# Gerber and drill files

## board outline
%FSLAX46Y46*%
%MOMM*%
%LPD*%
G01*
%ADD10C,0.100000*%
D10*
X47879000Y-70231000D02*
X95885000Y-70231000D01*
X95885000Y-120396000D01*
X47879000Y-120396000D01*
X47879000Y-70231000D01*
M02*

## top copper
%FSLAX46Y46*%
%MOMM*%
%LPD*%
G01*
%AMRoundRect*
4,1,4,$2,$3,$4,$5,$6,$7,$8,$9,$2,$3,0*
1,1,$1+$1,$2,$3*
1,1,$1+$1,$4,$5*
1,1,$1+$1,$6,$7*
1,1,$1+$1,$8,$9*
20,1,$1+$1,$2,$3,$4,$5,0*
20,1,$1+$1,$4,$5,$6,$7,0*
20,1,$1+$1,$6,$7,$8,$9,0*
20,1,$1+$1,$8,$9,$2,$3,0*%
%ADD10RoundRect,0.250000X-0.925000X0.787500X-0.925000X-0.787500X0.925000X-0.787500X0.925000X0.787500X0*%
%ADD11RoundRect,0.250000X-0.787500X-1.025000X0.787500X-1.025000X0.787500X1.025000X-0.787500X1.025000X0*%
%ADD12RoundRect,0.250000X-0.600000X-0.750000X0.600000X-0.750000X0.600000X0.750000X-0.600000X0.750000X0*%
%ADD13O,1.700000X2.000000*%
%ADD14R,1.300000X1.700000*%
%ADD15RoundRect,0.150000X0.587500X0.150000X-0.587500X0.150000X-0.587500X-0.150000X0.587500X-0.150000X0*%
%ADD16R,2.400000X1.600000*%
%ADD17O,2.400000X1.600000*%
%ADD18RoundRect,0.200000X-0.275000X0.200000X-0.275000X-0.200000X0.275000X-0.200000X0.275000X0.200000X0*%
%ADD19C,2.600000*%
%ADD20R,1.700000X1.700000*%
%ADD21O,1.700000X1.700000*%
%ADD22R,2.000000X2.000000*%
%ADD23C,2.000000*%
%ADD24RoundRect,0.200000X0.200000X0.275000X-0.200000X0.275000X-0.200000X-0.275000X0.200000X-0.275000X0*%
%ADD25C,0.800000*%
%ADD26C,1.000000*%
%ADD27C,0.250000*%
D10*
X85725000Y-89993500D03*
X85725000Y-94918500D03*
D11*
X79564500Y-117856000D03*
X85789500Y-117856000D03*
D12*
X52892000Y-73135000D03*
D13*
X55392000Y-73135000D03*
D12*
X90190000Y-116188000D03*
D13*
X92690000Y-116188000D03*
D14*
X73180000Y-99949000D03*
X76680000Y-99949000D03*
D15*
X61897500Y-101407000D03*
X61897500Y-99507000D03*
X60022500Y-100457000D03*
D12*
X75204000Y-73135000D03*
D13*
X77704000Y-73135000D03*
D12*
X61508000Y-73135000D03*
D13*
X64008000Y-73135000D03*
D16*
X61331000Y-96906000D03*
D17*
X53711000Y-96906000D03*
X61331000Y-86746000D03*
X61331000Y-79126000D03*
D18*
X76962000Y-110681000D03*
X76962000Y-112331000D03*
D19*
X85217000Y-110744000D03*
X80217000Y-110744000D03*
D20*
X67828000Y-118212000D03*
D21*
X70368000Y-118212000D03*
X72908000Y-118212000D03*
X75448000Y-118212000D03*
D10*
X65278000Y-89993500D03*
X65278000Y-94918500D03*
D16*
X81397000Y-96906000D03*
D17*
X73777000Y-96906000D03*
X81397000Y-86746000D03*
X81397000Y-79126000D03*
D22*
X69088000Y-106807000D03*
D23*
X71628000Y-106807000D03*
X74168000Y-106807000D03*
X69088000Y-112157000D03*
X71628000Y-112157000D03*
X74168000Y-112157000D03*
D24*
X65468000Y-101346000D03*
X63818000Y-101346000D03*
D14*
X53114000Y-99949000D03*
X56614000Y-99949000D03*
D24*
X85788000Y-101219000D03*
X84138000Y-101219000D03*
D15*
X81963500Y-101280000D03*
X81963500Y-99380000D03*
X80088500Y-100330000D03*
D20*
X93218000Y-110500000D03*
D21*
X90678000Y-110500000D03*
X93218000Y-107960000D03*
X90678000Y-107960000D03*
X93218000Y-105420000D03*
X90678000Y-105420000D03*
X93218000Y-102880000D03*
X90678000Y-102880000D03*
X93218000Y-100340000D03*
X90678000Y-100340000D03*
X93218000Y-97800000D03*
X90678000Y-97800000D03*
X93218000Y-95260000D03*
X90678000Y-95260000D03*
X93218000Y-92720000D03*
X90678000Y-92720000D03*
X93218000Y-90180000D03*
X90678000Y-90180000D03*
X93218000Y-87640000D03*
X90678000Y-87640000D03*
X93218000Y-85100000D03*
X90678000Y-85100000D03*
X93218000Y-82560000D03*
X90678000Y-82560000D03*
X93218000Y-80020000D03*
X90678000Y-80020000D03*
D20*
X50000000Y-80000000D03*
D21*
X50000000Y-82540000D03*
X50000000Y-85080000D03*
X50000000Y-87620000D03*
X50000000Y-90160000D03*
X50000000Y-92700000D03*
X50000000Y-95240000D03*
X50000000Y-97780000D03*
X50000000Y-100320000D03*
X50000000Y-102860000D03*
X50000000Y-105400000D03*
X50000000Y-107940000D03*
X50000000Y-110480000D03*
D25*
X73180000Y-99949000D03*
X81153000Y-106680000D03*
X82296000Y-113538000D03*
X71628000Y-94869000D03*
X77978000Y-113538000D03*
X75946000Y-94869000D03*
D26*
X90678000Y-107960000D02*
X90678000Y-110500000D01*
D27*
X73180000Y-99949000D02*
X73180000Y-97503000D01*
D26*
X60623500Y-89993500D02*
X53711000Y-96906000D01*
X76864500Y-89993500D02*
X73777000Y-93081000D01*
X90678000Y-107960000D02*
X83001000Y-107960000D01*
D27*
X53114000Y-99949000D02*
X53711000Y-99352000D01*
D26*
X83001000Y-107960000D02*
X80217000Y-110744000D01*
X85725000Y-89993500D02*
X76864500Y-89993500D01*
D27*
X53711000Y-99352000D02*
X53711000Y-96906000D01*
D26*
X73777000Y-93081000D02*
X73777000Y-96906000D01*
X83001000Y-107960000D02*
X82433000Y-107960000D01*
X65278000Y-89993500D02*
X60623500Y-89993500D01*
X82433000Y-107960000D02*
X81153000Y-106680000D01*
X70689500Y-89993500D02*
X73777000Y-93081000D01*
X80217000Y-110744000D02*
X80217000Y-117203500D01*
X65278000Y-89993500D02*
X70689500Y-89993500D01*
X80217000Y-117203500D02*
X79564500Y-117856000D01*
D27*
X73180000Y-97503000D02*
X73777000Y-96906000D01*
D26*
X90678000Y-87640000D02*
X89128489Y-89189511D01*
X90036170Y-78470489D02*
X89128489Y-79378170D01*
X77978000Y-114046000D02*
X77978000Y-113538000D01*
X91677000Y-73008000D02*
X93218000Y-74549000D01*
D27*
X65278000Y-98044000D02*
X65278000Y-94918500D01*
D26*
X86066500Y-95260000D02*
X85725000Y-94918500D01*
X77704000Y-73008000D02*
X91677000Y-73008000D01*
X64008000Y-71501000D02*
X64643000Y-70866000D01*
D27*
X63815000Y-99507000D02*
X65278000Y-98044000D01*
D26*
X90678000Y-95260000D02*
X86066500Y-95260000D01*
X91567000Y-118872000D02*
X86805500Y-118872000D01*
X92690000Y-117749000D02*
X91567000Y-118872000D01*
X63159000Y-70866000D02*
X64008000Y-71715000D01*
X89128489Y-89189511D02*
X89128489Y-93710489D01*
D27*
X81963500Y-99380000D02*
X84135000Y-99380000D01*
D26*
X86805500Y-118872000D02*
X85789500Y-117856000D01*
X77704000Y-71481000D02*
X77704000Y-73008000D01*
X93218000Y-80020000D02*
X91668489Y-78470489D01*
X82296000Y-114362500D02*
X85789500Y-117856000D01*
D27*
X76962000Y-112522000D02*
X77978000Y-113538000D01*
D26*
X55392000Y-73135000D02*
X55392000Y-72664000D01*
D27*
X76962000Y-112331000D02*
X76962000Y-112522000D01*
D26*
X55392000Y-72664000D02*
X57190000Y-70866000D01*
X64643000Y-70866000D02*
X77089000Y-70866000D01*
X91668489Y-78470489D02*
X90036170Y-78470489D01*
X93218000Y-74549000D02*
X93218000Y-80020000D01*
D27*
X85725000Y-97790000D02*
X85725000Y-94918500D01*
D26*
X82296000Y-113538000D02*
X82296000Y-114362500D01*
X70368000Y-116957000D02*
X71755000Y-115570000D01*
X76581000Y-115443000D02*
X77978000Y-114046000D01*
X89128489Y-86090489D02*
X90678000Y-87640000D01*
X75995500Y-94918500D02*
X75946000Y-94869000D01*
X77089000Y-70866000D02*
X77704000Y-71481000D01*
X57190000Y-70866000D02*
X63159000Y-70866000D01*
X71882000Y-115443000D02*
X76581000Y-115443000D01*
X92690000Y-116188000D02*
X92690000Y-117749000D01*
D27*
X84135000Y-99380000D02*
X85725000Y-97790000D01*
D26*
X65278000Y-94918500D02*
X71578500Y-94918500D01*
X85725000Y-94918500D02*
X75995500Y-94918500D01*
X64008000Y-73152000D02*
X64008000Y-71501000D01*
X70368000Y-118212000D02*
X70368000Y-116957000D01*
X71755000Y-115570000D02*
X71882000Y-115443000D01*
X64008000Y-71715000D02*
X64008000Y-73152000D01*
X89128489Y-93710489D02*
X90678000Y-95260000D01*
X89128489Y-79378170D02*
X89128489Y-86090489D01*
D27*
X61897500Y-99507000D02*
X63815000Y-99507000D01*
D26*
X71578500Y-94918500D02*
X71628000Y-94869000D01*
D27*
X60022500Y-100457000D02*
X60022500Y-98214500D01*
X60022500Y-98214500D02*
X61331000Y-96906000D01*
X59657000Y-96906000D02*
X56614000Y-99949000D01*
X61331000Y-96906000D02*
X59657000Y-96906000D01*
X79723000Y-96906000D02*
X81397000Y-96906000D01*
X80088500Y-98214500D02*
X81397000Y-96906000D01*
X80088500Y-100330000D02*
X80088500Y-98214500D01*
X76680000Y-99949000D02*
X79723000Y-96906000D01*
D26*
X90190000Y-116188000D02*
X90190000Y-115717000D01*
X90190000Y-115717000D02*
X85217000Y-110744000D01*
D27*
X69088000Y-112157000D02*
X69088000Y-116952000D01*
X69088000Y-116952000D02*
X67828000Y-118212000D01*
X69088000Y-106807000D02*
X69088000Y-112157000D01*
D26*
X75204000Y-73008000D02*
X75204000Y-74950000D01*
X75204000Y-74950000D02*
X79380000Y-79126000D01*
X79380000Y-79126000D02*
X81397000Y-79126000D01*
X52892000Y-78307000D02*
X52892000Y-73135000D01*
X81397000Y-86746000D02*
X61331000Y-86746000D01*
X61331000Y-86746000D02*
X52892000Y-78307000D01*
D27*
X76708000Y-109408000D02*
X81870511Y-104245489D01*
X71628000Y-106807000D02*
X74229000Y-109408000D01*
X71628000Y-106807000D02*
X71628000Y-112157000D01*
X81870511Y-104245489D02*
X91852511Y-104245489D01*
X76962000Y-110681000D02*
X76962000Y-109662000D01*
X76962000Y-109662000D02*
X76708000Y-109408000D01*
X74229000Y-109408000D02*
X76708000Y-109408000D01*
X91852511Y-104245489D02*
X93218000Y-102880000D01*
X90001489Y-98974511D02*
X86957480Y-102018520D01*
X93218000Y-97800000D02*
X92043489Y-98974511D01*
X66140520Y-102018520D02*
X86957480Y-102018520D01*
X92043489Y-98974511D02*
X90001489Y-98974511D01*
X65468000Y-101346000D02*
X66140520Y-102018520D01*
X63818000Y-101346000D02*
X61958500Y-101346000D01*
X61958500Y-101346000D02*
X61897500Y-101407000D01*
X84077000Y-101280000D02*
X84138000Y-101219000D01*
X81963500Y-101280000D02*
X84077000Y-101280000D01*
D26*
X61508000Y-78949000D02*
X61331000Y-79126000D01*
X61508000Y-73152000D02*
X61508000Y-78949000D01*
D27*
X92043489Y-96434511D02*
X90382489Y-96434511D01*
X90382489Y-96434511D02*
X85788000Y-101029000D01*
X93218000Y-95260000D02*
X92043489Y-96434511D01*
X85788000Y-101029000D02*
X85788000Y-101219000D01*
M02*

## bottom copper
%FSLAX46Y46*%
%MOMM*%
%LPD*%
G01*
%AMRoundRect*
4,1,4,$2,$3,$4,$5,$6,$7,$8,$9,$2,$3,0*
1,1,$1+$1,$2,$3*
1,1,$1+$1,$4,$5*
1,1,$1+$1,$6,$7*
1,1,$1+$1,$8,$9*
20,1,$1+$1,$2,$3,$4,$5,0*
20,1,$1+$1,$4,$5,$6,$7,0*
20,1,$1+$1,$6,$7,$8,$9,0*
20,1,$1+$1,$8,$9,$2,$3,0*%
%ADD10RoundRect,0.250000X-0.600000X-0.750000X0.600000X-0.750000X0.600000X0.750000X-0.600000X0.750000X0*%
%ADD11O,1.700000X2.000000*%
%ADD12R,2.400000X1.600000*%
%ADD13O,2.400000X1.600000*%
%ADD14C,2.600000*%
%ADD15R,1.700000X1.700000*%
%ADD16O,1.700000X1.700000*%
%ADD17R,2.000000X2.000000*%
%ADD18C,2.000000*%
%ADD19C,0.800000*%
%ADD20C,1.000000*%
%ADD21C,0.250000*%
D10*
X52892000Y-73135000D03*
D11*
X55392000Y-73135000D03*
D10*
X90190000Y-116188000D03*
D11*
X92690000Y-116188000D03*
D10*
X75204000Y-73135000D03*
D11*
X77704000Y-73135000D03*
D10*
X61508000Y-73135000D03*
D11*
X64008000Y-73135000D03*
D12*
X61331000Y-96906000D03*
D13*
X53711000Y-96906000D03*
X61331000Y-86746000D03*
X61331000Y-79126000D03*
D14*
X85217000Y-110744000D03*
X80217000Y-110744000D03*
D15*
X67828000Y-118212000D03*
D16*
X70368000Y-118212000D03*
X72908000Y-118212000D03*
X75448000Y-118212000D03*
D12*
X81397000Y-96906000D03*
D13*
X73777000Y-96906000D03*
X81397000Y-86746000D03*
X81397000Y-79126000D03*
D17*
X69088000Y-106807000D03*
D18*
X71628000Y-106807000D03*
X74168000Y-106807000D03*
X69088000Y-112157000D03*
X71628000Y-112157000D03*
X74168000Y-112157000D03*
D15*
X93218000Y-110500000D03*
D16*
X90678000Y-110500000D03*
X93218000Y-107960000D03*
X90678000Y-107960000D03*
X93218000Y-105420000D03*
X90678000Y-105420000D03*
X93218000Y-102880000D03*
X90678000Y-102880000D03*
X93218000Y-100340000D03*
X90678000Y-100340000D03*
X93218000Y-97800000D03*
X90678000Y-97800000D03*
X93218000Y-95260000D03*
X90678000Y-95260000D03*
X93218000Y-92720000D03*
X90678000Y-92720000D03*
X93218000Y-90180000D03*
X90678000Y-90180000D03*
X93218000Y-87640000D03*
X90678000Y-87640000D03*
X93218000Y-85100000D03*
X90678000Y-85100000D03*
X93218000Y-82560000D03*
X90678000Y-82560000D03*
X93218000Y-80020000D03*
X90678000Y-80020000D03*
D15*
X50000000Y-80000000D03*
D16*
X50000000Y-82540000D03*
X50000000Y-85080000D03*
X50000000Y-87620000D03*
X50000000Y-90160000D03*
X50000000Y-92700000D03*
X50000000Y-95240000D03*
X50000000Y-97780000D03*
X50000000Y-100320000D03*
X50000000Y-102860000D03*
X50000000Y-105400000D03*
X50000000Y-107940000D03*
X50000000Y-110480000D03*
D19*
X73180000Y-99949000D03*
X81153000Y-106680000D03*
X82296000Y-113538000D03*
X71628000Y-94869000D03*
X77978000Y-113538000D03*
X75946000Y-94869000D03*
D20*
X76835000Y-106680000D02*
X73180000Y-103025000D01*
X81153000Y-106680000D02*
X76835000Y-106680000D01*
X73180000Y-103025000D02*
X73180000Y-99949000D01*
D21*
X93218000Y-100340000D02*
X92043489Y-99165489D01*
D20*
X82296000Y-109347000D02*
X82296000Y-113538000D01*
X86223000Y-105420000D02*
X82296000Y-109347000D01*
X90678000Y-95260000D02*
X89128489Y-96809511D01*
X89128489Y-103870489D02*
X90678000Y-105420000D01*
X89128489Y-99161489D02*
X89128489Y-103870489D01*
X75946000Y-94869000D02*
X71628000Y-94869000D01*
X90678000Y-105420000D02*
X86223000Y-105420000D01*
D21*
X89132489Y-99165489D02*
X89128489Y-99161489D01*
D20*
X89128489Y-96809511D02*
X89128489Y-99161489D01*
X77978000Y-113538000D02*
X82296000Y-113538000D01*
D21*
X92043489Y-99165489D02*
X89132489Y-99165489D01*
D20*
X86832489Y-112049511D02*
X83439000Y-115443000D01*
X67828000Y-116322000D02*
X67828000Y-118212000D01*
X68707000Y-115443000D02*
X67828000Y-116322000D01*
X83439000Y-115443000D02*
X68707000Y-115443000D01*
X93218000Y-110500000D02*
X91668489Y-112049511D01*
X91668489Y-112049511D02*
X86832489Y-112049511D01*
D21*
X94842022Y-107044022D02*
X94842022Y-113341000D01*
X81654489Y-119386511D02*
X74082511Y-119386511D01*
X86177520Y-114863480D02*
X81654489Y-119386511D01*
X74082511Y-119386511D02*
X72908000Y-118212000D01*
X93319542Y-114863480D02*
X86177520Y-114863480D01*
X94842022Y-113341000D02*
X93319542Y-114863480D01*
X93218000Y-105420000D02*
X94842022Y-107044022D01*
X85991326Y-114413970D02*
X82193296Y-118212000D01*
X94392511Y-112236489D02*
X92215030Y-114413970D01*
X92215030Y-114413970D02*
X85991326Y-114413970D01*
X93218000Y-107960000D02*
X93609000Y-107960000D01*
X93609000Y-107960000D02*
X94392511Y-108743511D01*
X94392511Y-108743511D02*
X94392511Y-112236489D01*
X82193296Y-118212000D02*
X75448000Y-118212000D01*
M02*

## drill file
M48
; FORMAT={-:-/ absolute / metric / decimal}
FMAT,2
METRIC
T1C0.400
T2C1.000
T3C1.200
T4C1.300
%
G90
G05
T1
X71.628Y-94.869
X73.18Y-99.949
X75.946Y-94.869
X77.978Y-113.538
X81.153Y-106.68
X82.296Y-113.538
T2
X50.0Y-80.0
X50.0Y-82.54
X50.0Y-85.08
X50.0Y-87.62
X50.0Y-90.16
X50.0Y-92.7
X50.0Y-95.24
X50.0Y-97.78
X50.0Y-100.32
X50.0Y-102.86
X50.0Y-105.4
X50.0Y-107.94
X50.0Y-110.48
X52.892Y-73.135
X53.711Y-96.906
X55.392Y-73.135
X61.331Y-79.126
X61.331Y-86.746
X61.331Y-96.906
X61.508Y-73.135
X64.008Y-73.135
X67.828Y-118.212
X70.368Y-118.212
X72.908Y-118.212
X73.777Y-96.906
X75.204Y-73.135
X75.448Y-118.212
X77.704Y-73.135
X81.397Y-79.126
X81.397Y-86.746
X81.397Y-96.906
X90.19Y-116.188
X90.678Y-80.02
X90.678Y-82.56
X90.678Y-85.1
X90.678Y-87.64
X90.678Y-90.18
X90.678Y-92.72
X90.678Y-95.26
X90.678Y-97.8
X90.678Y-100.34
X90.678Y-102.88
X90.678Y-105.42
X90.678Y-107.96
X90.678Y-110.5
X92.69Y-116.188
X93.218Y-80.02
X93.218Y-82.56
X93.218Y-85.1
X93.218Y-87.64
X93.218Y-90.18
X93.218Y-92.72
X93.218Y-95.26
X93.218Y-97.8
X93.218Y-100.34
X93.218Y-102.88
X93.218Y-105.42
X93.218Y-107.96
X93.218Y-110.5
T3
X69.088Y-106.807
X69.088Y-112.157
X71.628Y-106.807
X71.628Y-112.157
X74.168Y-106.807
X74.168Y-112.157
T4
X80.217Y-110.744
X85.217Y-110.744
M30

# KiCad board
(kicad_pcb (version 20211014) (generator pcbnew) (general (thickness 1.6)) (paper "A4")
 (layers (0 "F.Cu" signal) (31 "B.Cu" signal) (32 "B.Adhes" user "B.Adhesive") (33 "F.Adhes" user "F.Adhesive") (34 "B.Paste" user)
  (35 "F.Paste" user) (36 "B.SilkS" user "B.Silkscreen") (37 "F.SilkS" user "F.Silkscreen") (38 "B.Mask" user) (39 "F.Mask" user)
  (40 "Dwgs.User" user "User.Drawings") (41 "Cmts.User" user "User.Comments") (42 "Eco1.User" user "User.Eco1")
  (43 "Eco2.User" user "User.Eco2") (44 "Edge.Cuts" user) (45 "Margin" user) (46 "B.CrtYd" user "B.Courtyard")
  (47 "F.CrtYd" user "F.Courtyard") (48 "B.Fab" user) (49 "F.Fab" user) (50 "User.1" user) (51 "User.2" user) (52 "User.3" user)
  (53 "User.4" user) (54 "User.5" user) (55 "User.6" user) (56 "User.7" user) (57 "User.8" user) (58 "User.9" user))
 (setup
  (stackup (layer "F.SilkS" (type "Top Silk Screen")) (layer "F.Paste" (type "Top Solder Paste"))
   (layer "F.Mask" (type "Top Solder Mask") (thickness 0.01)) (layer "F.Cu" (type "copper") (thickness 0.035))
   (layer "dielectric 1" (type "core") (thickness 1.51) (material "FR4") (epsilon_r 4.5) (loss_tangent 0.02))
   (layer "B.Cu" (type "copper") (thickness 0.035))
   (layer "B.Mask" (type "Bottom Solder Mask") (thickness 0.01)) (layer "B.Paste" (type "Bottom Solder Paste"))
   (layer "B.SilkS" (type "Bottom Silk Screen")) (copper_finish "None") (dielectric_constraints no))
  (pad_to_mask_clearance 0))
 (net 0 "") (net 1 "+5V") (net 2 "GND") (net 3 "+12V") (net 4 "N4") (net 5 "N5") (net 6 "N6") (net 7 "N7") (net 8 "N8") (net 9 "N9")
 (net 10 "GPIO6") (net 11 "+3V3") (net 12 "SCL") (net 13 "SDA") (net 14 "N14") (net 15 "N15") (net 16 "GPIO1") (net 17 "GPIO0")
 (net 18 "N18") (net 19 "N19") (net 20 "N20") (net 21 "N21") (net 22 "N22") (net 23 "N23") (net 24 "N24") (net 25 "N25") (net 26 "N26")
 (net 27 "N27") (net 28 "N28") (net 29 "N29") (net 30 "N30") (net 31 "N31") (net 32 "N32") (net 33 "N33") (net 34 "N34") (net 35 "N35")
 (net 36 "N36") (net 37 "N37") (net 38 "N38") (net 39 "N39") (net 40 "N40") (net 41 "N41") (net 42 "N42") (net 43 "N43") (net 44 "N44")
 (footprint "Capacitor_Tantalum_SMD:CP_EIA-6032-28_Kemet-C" (layer "F.Cu") (at 85.725 92.456 -90)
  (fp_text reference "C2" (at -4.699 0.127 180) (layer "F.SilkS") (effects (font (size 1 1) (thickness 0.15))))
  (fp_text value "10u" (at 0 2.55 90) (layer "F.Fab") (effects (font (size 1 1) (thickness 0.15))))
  (pad "1" smd roundrect (at -2.4625 0 270) (size 2.075 2.35) (layers "F.Cu" "F.Paste" "F.Mask") (roundrect_rratio 0.1204819277)
   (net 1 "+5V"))
  (pad "2" smd roundrect (at 2.4625 0 270) (size 2.075 2.35) (layers "F.Cu" "F.Paste" "F.Mask") (roundrect_rratio 0.1204819277)
   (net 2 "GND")))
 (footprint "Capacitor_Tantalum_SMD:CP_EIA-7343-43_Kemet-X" (layer "F.Cu") (at 82.677 117.856)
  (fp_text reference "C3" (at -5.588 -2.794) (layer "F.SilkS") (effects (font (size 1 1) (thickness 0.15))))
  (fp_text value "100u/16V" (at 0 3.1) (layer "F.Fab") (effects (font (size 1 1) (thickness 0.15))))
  (pad "1" smd roundrect (at -3.1125 0) (size 2.075 2.55) (layers "F.Cu" "F.Paste" "F.Mask") (roundrect_rratio 0.1204819277) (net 1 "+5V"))
  (pad "2" smd roundrect (at 3.1125 0) (size 2.075 2.55) (layers "F.Cu" "F.Paste" "F.Mask") (roundrect_rratio 0.1204819277) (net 2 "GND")))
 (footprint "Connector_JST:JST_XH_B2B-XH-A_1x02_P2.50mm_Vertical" (layer "F.Cu") (at 52.892 73.135)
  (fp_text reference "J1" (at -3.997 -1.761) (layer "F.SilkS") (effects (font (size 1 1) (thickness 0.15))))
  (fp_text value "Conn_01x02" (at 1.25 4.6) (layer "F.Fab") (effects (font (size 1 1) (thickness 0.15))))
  (pad "1" thru_hole roundrect (at 0 0) (size 1.7 2) (drill 1) (layers *.Cu *.Mask) (roundrect_rratio 0.1470588235) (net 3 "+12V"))
  (pad "2" thru_hole oval (at 2.5 0) (size 1.7 2) (drill 1) (layers *.Cu *.Mask) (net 2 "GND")))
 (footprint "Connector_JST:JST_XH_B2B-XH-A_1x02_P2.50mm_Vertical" (layer "F.Cu") (at 90.19 116.188)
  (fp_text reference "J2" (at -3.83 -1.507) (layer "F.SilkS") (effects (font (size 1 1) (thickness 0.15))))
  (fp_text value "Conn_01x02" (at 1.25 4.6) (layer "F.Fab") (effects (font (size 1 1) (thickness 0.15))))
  (pad "1" thru_hole roundrect (at 0 0) (size 1.7 2) (drill 1) (layers *.Cu *.Mask) (roundrect_rratio 0.147059) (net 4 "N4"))
  (pad "2" thru_hole oval (at 2.5 0) (size 1.7 2) (drill 1) (layers *.Cu *.Mask) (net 2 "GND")))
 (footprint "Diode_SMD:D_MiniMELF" (layer "F.Cu") (at 74.93 99.949)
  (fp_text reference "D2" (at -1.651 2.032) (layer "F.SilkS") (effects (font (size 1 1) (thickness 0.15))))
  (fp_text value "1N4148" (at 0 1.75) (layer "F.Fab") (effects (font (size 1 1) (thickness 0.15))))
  (pad "1" smd rect (at -1.75 0) (size 1.3 1.7) (layers "F.Cu" "F.Paste" "F.Mask") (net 1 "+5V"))
  (pad "2" smd rect (at 1.75 0) (size 1.3 1.7) (layers "F.Cu" "F.Paste" "F.Mask") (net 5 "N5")))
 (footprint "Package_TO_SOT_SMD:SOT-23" (layer "F.Cu") (at 60.96 100.457 180)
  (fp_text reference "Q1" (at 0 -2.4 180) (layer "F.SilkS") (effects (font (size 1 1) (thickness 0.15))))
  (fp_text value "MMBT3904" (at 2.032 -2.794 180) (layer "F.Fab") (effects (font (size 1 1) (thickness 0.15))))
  (pad "1" smd roundrect (at -0.9375 -0.95 180) (size 1.475 0.6) (layers "F.Cu" "F.Paste" "F.Mask") (roundrect_rratio 0.25) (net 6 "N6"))
  (pad "2" smd roundrect (at -0.9375 0.95 180) (size 1.475 0.6) (layers "F.Cu" "F.Paste" "F.Mask") (roundrect_rratio 0.25) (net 2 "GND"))
  (pad "3" smd roundrect (at 0.9375 0 180) (size 1.475 0.6) (layers "F.Cu" "F.Paste" "F.Mask") (roundrect_rratio 0.25) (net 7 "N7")))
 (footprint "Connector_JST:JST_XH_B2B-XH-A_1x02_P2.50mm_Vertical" (layer "F.Cu") (at 75.204 73.135)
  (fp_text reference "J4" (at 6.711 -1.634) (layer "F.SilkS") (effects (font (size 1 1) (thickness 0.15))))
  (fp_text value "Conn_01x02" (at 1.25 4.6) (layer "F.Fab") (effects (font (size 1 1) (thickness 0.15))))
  (pad "1" thru_hole roundrect (at 0 0) (size 1.7 2) (drill 1) (layers *.Cu *.Mask) (roundrect_rratio 0.1470588235) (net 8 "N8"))
  (pad "2" thru_hole oval (at 2.5 0) (size 1.7 2) (drill 1) (layers *.Cu *.Mask) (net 2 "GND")))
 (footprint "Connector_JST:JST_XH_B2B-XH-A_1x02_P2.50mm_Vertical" (layer "F.Cu") (at 61.508 73.135)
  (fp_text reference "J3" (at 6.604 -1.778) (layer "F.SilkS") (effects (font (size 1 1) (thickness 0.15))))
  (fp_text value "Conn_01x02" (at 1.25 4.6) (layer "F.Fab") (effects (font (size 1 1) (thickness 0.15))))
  (pad "1" thru_hole roundrect (at 0 0) (size 1.7 2) (drill 1) (layers *.Cu *.Mask) (roundrect_rratio 0.147059) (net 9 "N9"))
  (pad "2" thru_hole oval (at 2.5 0) (size 1.7 2) (drill 1) (layers *.Cu *.Mask) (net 2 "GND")))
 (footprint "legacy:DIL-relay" (layer "F.Cu") (at 61.331 96.906 180)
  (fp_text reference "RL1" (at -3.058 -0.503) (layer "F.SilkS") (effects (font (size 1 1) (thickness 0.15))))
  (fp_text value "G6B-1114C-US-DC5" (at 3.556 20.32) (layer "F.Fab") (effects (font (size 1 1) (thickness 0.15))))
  (pad "1" thru_hole rect locked (at 0 0 180) (size 2.4 1.6) (drill 1) (layers *.Cu *.Mask) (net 7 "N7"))
  (pad "2" thru_hole oval locked (at 7.62 0 180) (size 2.4 1.6) (drill 1) (layers *.Cu *.Mask) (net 1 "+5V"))
  (pad "3" thru_hole oval locked (at 0 10.16 180) (size 2.4 1.6) (drill 1) (layers *.Cu *.Mask) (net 3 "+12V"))
  (pad "4" thru_hole oval locked (at 0 17.78 180) (size 2.4 1.6) (drill 1) (layers *.Cu *.Mask) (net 9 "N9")))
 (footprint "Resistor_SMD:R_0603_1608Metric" (layer "F.Cu") (at 76.962 111.506 -90)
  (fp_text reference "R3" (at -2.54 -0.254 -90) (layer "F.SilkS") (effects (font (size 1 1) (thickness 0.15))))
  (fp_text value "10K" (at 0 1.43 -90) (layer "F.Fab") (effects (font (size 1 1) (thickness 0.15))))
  (pad "1" smd roundrect (at -0.825 0 270) (size 0.8 0.95) (layers "F.Cu" "F.Paste" "F.Mask") (roundrect_rratio 0.25) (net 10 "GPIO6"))
  (pad "2" smd roundrect (at 0.825 0 270) (size 0.8 0.95) (layers "F.Cu" "F.Paste" "F.Mask") (roundrect_rratio 0.25) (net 2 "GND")))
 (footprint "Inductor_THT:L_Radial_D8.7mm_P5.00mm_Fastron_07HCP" (layer "F.Cu") (at 85.217 110.744 180)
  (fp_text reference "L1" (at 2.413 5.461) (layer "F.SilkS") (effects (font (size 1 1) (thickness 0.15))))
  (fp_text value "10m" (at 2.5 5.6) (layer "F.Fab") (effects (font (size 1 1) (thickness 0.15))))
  (pad "1" thru_hole circle (at 0 0 180) (size 2.6 2.6) (drill 1.3) (layers *.Cu *.Mask) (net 4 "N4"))
  (pad "2" thru_hole circle (at 5 0 180) (size 2.6 2.6) (drill 1.3) (layers *.Cu *.Mask) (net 1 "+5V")))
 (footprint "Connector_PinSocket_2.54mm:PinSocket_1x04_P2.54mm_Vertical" (layer "F.Cu") (at 67.828 118.212 90)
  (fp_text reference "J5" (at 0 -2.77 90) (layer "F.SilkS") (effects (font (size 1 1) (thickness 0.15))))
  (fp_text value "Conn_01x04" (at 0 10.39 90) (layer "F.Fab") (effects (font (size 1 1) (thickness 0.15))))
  (pad "1" thru_hole rect (at 0 0 90) (size 1.7 1.7) (drill 1) (layers *.Cu *.Mask) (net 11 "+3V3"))
  (pad "2" thru_hole oval (at 0 2.54 90) (size 1.7 1.7) (drill 1) (layers *.Cu *.Mask) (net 2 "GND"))
  (pad "3" thru_hole oval (at 0 5.08 90) (size 1.7 1.7) (drill 1) (layers *.Cu *.Mask) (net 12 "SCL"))
  (pad "4" thru_hole oval (at 0 7.62 90) (size 1.7 1.7) (drill 1) (layers *.Cu *.Mask) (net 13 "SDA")))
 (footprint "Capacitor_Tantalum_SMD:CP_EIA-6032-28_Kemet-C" (layer "F.Cu") (at 65.278 92.456 -90)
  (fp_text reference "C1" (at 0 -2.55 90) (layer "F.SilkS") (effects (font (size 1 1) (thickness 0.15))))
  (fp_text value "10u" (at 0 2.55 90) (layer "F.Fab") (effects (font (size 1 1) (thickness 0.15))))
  (pad "1" smd roundrect (at -2.4625 0 270) (size 2.075 2.35) (layers "F.Cu" "F.Paste" "F.Mask") (roundrect_rratio 0.1204819277)
   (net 1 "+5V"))
  (pad "2" smd roundrect (at 2.4625 0 270) (size 2.075 2.35) (layers "F.Cu" "F.Paste" "F.Mask") (roundrect_rratio 0.1204819277)
   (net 2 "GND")))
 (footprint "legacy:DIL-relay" (layer "F.Cu") (at 81.397 96.906 180)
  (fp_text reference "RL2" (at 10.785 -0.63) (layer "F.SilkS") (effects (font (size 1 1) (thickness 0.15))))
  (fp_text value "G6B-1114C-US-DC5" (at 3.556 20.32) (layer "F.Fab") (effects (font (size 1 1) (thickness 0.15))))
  (pad "1" thru_hole rect locked (at 0 0 180) (size 2.4 1.6) (drill 1) (layers *.Cu *.Mask) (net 5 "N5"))
  (pad "2" thru_hole oval locked (at 7.62 0 180) (size 2.4 1.6) (drill 1) (layers *.Cu *.Mask) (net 1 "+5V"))
  (pad "3" thru_hole oval locked (at 0 10.16 180) (size 2.4 1.6) (drill 1) (layers *.Cu *.Mask) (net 3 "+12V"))
  (pad "4" thru_hole oval locked (at 0 17.78 180) (size 2.4 1.6) (drill 1) (layers *.Cu *.Mask) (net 8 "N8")))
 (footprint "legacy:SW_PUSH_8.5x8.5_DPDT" (layer "F.Cu") (at 69.088 106.807)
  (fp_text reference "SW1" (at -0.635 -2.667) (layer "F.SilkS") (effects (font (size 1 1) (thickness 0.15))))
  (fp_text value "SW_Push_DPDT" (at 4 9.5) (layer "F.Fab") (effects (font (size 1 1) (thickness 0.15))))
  (pad "1" thru_hole rect locked (at 0 0) (size 2 2) (drill 1.2) (layers *.Cu *.Mask) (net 11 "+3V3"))
  (pad "2" thru_hole circle locked (at 2.54 0) (size 2 2) (drill 1.2) (layers *.Cu *.Mask) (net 10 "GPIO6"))
  (pad "3" thru_hole circle locked (at 5.08 0) (size 2 2) (drill 1.2) (layers *.Cu *.Mask) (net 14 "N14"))
  (pad "4" thru_hole circle locked (at 0 5.35) (size 2 2) (drill 1.2) (layers *.Cu *.Mask) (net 11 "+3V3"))
  (pad "5" thru_hole circle locked (at 2.54 5.35) (size 2 2) (drill 1.2) (layers *.Cu *.Mask) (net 10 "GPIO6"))
  (pad "6" thru_hole circle locked (at 5.08 5.35) (size 2 2) (drill 1.2) (layers *.Cu *.Mask) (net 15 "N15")))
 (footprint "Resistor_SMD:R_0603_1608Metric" (layer "F.Cu") (at 64.643 101.346 180)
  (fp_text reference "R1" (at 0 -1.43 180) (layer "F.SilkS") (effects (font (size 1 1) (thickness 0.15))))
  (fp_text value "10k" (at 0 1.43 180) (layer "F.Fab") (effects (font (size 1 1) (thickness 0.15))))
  (pad "1" smd roundrect (at -0.825 0 180) (size 0.8 0.95) (layers "F.Cu" "F.Paste" "F.Mask") (roundrect_rratio 0.25) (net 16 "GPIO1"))
  (pad "2" smd roundrect (at 0.825 0 180) (size 0.8 0.95) (layers "F.Cu" "F.Paste" "F.Mask") (roundrect_rratio 0.25) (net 6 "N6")))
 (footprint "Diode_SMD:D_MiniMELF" (layer "F.Cu") (at 54.864 99.949)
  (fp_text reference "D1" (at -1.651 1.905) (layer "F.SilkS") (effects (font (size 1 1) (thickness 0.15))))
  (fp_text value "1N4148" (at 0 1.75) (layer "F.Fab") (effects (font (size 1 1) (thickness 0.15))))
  (pad "1" smd rect (at -1.75 0) (size 1.3 1.7) (layers "F.Cu" "F.Paste" "F.Mask") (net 1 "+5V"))
  (pad "2" smd rect (at 1.75 0) (size 1.3 1.7) (layers "F.Cu" "F.Paste" "F.Mask") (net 7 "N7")))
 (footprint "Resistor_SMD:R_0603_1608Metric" (layer "F.Cu") (at 84.963 101.219 180)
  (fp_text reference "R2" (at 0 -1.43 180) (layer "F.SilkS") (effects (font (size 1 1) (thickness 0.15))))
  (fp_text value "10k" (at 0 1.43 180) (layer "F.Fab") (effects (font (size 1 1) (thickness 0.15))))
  (pad "1" smd roundrect (at -0.825 0 180) (size 0.8 0.95) (layers "F.Cu" "F.Paste" "F.Mask") (roundrect_rratio 0.25) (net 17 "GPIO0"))
  (pad "2" smd roundrect (at 0.825 0 180) (size 0.8 0.95) (layers "F.Cu" "F.Paste" "F.Mask") (roundrect_rratio 0.25) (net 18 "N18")))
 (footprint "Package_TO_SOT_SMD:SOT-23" (layer "F.Cu") (at 81.026 100.33 180)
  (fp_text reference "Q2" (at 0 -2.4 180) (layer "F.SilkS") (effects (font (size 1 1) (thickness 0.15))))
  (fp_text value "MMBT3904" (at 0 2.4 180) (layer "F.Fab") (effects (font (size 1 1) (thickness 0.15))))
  (pad "1" smd roundrect (at -0.9375 -0.95 180) (size 1.475 0.6) (layers "F.Cu" "F.Paste" "F.Mask") (roundrect_rratio 0.25) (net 18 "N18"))
  (pad "2" smd roundrect (at -0.9375 0.95 180) (size 1.475 0.6) (layers "F.Cu" "F.Paste" "F.Mask") (roundrect_rratio 0.25) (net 2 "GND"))
  (pad "3" smd roundrect (at 0.9375 0 180) (size 1.475 0.6) (layers "F.Cu" "F.Paste" "F.Mask") (roundrect_rratio 0.25) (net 5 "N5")))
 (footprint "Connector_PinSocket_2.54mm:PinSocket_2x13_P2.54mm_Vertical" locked (layer "B.Cu") (at 93.218 110.5)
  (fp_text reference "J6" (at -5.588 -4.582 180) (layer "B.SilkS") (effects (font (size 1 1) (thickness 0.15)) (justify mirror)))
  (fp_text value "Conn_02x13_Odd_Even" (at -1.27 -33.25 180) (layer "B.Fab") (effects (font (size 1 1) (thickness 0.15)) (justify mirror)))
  (pad "1" thru_hole rect locked (at 0 0) (size 1.7 1.7) (drill 1) (layers *.Cu *.Mask) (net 11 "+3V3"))
  (pad "2" thru_hole oval locked (at -2.54 0) (size 1.7 1.7) (drill 1) (layers *.Cu *.Mask) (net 1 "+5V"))
  (pad "3" thru_hole oval locked (at 0 -2.54) (size 1.7 1.7) (drill 1) (layers *.Cu *.Mask) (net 13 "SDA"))
  (pad "4" thru_hole oval locked (at -2.54 -2.54) (size 1.7 1.7) (drill 1) (layers *.Cu *.Mask) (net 1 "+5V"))
  (pad "5" thru_hole oval locked (at 0 -5.08) (size 1.7 1.7) (drill 1) (layers *.Cu *.Mask) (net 12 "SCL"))
  (pad "6" thru_hole oval locked (at -2.54 -5.08) (size 1.7 1.7) (drill 1) (layers *.Cu *.Mask) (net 2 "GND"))
  (pad "7" thru_hole oval locked (at 0 -7.62) (size 1.7 1.7) (drill 1) (layers *.Cu *.Mask) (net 10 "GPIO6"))
  (pad "8" thru_hole oval locked (at -2.54 -7.62) (size 1.7 1.7) (drill 1) (layers *.Cu *.Mask) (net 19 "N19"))
  (pad "9" thru_hole oval locked (at 0 -10.16) (size 1.7 1.7) (drill 1) (layers *.Cu *.Mask) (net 2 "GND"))
  (pad "10" thru_hole oval locked (at -2.54 -10.16) (size 1.7 1.7) (drill 1) (layers *.Cu *.Mask) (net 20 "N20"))
  (pad "11" thru_hole oval locked (at 0 -12.7) (size 1.7 1.7) (drill 1) (layers *.Cu *.Mask) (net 16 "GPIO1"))
  (pad "12" thru_hole oval locked (at -2.54 -12.7) (size 1.7 1.7) (drill 1) (layers *.Cu *.Mask) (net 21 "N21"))
  (pad "13" thru_hole oval locked (at 0 -15.24) (size 1.7 1.7) (drill 1) (layers *.Cu *.Mask) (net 17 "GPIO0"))
  (pad "14" thru_hole oval locked (at -2.54 -15.24) (size 1.7 1.7) (drill 1) (layers *.Cu *.Mask) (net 2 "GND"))
  (pad "15" thru_hole oval locked (at 0 -17.78) (size 1.7 1.7) (drill 1) (layers *.Cu *.Mask) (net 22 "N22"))
  (pad "16" thru_hole oval locked (at -2.54 -17.78) (size 1.7 1.7) (drill 1) (layers *.Cu *.Mask) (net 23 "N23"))
  (pad "17" thru_hole oval locked (at 0 -20.32) (size 1.7 1.7) (drill 1) (layers *.Cu *.Mask) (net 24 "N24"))
  (pad "18" thru_hole oval locked (at -2.54 -20.32) (size 1.7 1.7) (drill 1) (layers *.Cu *.Mask) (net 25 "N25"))
  (pad "19" thru_hole oval locked (at 0 -22.86) (size 1.7 1.7) (drill 1) (layers *.Cu *.Mask) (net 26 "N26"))
  (pad "20" thru_hole oval locked (at -2.54 -22.86) (size 1.7 1.7) (drill 1) (layers *.Cu *.Mask) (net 2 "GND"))
  (pad "21" thru_hole oval locked (at 0 -25.4) (size 1.7 1.7) (drill 1) (layers *.Cu *.Mask) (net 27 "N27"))
  (pad "22" thru_hole oval locked (at -2.54 -25.4) (size 1.7 1.7) (drill 1) (layers *.Cu *.Mask) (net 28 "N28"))
  (pad "23" thru_hole oval locked (at 0 -27.94) (size 1.7 1.7) (drill 1) (layers *.Cu *.Mask) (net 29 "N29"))
  (pad "24" thru_hole oval locked (at -2.54 -27.94) (size 1.7 1.7) (drill 1) (layers *.Cu *.Mask) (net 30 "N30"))
  (pad "25" thru_hole oval locked (at 0 -30.48) (size 1.7 1.7) (drill 1) (layers *.Cu *.Mask) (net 2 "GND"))
  (pad "26" thru_hole oval locked (at -2.54 -30.48) (size 1.7 1.7) (drill 1) (layers *.Cu *.Mask) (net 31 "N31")))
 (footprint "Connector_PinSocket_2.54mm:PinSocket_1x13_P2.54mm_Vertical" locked (layer "B.Cu") (at 50 80 180)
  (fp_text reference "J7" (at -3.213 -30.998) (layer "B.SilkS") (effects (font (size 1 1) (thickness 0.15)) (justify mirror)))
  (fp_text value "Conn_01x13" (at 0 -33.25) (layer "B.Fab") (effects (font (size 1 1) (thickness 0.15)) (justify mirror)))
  (pad "1" thru_hole rect locked (at 0 0 180) (size 1.7 1.7) (drill 1) (layers *.Cu *.Mask) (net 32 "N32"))
  (pad "2" thru_hole oval locked (at 0 -2.54 180) (size 1.7 1.7) (drill 1) (layers *.Cu *.Mask) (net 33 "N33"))
  (pad "3" thru_hole oval locked (at 0 -5.08 180) (size 1.7 1.7) (drill 1) (layers *.Cu *.Mask) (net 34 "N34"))
  (pad "4" thru_hole oval locked (at 0 -7.62 180) (size 1.7 1.7) (drill 1) (layers *.Cu *.Mask) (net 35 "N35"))
  (pad "5" thru_hole oval locked (at 0 -10.16 180) (size 1.7 1.7) (drill 1) (layers *.Cu *.Mask) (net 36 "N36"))
  (pad "6" thru_hole oval locked (at 0 -12.7 180) (size 1.7 1.7) (drill 1) (layers *.Cu *.Mask) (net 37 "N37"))
  (pad "7" thru_hole oval locked (at 0 -15.24 180) (size 1.7 1.7) (drill 1) (layers *.Cu *.Mask) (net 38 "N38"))
  (pad "8" thru_hole oval locked (at 0 -17.78 180) (size 1.7 1.7) (drill 1) (layers *.Cu *.Mask) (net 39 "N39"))
  (pad "9" thru_hole oval locked (at 0 -20.32 180) (size 1.7 1.7) (drill 1) (layers *.Cu *.Mask) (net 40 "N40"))
  (pad "10" thru_hole oval locked (at 0 -22.86 180) (size 1.7 1.7) (drill 1) (layers *.Cu *.Mask) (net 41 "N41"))
  (pad "11" thru_hole oval locked (at 0 -25.4 180) (size 1.7 1.7) (drill 1) (layers *.Cu *.Mask) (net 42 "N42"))
  (pad "12" thru_hole oval locked (at 0 -27.94 180) (size 1.7 1.7) (drill 1) (layers *.Cu *.Mask) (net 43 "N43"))
  (pad "13" thru_hole oval locked (at 0 -30.48 180) (size 1.7 1.7) (drill 1) (layers *.Cu *.Mask) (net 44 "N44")))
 (gr_rect (start 47.879 70.231) (end 95.885 120.396) (layer "Edge.Cuts") (width 0.1) (fill none))
 (segment (start 90.678 107.96) (end 90.678 110.5) (width 1) (layer "F.Cu") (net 1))
 (segment (start 73.18 99.949) (end 73.18 97.503) (width 0.25) (layer "F.Cu") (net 1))
 (segment (start 60.6235 89.9935) (end 53.711 96.906) (width 1) (layer "F.Cu") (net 1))
 (segment (start 76.8645 89.9935) (end 73.777 93.081) (width 1) (layer "F.Cu") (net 1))
 (segment (start 90.678 107.96) (end 83.001 107.96) (width 1) (layer "F.Cu") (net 1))
 (segment (start 53.114 99.949) (end 53.711 99.352) (width 0.25) (layer "F.Cu") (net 1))
 (segment (start 83.001 107.96) (end 80.217 110.744) (width 1) (layer "F.Cu") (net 1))
 (segment (start 85.725 89.9935) (end 76.8645 89.9935) (width 1) (layer "F.Cu") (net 1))
 (segment (start 53.711 99.352) (end 53.711 96.906) (width 0.25) (layer "F.Cu") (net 1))
 (segment (start 73.777 93.081) (end 73.777 96.906) (width 1) (layer "F.Cu") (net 1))
 (segment (start 83.001 107.96) (end 82.433 107.96) (width 1) (layer "F.Cu") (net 1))
 (segment (start 65.278 89.9935) (end 60.6235 89.9935) (width 1) (layer "F.Cu") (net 1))
 (segment (start 82.433 107.96) (end 81.153 106.68) (width 1) (layer "F.Cu") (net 1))
 (segment (start 70.6895 89.9935) (end 73.777 93.081) (width 1) (layer "F.Cu") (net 1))
 (segment (start 80.217 110.744) (end 80.217 117.2035) (width 1) (layer "F.Cu") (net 1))
 (segment (start 65.278 89.9935) (end 70.6895 89.9935) (width 1) (layer "F.Cu") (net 1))
 (segment (start 80.217 117.2035) (end 79.5645 117.856) (width 1) (layer "F.Cu") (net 1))
 (segment (start 73.18 97.503) (end 73.777 96.906) (width 0.25) (layer "F.Cu") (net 1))
 (via (at 73.18 99.949) (size 0.8) (drill 0.4) (layers "F.Cu" "B.Cu") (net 1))
 (via (at 81.153 106.68) (size 0.8) (drill 0.4) (layers "F.Cu" "B.Cu") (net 1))
 (segment (start 76.835 106.68) (end 73.18 103.025) (width 1) (layer "B.Cu") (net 1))
 (segment (start 81.153 106.68) (end 76.835 106.68) (width 1) (layer "B.Cu") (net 1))
 (segment (start 73.18 103.025) (end 73.18 99.949) (width 1) (layer "B.Cu") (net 1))
 (segment (start 90.678 87.64) (end 89.128489 89.189511) (width 1) (layer "F.Cu") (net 2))
 (segment (start 90.03617 78.470489) (end 89.128489 79.37817) (width 1) (layer "F.Cu") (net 2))
 (segment (start 77.978 114.046) (end 77.978 113.538) (width 1) (layer "F.Cu") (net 2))
 (segment (start 91.677 73.008) (end 93.218 74.549) (width 1) (layer "F.Cu") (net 2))
 (segment (start 65.278 98.044) (end 65.278 94.9185) (width 0.25) (layer "F.Cu") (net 2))
 (segment (start 86.0665 95.26) (end 85.725 94.9185) (width 1) (layer "F.Cu") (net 2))
 (segment (start 77.704 73.008) (end 91.677 73.008) (width 1) (layer "F.Cu") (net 2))
 (segment (start 64.008 71.501) (end 64.643 70.866) (width 1) (layer "F.Cu") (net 2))
 (segment (start 63.815 99.507) (end 65.278 98.044) (width 0.25) (layer "F.Cu") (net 2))
 (segment (start 90.678 95.26) (end 86.0665 95.26) (width 1) (layer "F.Cu") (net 2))
 (segment (start 91.567 118.872) (end 86.8055 118.872) (width 1) (layer "F.Cu") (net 2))
 (segment (start 92.69 117.749) (end 91.567 118.872) (width 1) (layer "F.Cu") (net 2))
 (segment (start 63.159 70.866) (end 64.008 71.715) (width 1) (layer "F.Cu") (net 2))
 (segment (start 89.128489 89.189511) (end 89.128489 93.710489) (width 1) (layer "F.Cu") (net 2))
 (segment (start 81.9635 99.38) (end 84.135 99.38) (width 0.25) (layer "F.Cu") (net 2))
 (segment (start 86.8055 118.872) (end 85.7895 117.856) (width 1) (layer "F.Cu") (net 2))
 (segment (start 77.704 71.481) (end 77.704 73.008) (width 1) (layer "F.Cu") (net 2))
 (segment (start 93.218 80.02) (end 91.668489 78.470489) (width 1) (layer "F.Cu") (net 2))
 (segment (start 82.296 114.3625) (end 85.7895 117.856) (width 1) (layer "F.Cu") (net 2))
 (segment (start 76.962 112.522) (end 77.978 113.538) (width 0.25) (layer "F.Cu") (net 2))
 (segment (start 55.392 73.135) (end 55.392 72.664) (width 1) (layer "F.Cu") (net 2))
 (segment (start 76.962 112.331) (end 76.962 112.522) (width 0.25) (layer "F.Cu") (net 2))
 (segment (start 55.392 72.664) (end 57.19 70.866) (width 1) (layer "F.Cu") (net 2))
 (segment (start 64.643 70.866) (end 77.089 70.866) (width 1) (layer "F.Cu") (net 2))
 (segment (start 91.668489 78.470489) (end 90.03617 78.470489) (width 1) (layer "F.Cu") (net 2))
 (segment (start 93.218 74.549) (end 93.218 80.02) (width 1) (layer "F.Cu") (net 2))
 (segment (start 85.725 97.79) (end 85.725 94.9185) (width 0.25) (layer "F.Cu") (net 2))
 (segment (start 82.296 113.538) (end 82.296 114.3625) (width 1) (layer "F.Cu") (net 2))
 (segment (start 70.368 116.957) (end 71.755 115.57) (width 1) (layer "F.Cu") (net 2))
 (segment (start 76.581 115.443) (end 77.978 114.046) (width 1) (layer "F.Cu") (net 2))
 (segment (start 89.128489 86.090489) (end 90.678 87.64) (width 1) (layer "F.Cu") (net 2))
 (segment (start 75.9955 94.9185) (end 75.946 94.869) (width 1) (layer "F.Cu") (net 2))
 (segment (start 77.089 70.866) (end 77.704 71.481) (width 1) (layer "F.Cu") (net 2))
 (segment (start 57.19 70.866) (end 63.159 70.866) (width 1) (layer "F.Cu") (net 2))
 (segment (start 71.882 115.443) (end 76.581 115.443) (width 1) (layer "F.Cu") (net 2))
 (segment (start 92.69 116.188) (end 92.69 117.749) (width 1) (layer "F.Cu") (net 2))
 (segment (start 84.135 99.38) (end 85.725 97.79) (width 0.25) (layer "F.Cu") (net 2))
 (segment (start 65.278 94.9185) (end 71.5785 94.9185) (width 1) (layer "F.Cu") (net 2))
 (segment (start 85.725 94.9185) (end 75.9955 94.9185) (width 1) (layer "F.Cu") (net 2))
 (segment (start 64.008 73.152) (end 64.008 71.501) (width 1) (layer "F.Cu") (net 2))
 (segment (start 70.368 118.212) (end 70.368 116.957) (width 1) (layer "F.Cu") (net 2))
 (segment (start 71.755 115.57) (end 71.882 115.443) (width 1) (layer "F.Cu") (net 2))
 (segment (start 64.008 71.715) (end 64.008 73.152) (width 1) (layer "F.Cu") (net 2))
 (segment (start 89.128489 93.710489) (end 90.678 95.26) (width 1) (layer "F.Cu") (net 2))
 (segment (start 89.128489 79.37817) (end 89.128489 86.090489) (width 1) (layer "F.Cu") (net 2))
 (segment (start 61.8975 99.507) (end 63.815 99.507) (width 0.25) (layer "F.Cu") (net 2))
 (segment (start 71.5785 94.9185) (end 71.628 94.869) (width 1) (layer "F.Cu") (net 2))
 (via (at 82.296 113.538) (size 0.8) (drill 0.4) (layers "F.Cu" "B.Cu") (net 2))
 (via (at 71.628 94.869) (size 0.8) (drill 0.4) (layers "F.Cu" "B.Cu") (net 2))
 (via (at 77.978 113.538) (size 0.8) (drill 0.4) (layers "F.Cu" "B.Cu") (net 2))
 (via (at 75.946 94.869) (size 0.8) (drill 0.4) (layers "F.Cu" "B.Cu") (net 2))
 (segment (start 93.218 100.34) (end 92.043489 99.165489) (width 0.25) (layer "B.Cu") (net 2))
 (segment (start 82.296 109.347) (end 82.296 113.538) (width 1) (layer "B.Cu") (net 2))
 (segment (start 86.223 105.42) (end 82.296 109.347) (width 1) (layer "B.Cu") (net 2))
 (segment (start 90.678 95.26) (end 89.128489 96.809511) (width 1) (layer "B.Cu") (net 2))
 (segment (start 89.128489 103.870489) (end 90.678 105.42) (width 1) (layer "B.Cu") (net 2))
 (segment (start 89.128489 99.161489) (end 89.128489 103.870489) (width 1) (layer "B.Cu") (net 2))
 (segment (start 75.946 94.869) (end 71.628 94.869) (width 1) (layer "B.Cu") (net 2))
 (segment (start 90.678 105.42) (end 86.223 105.42) (width 1) (layer "B.Cu") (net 2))
 (segment (start 89.132489 99.165489) (end 89.128489 99.161489) (width 0.25) (layer "B.Cu") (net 2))
 (segment (start 89.128489 96.809511) (end 89.128489 99.161489) (width 1) (layer "B.Cu") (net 2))
 (segment (start 77.978 113.538) (end 82.296 113.538) (width 1) (layer "B.Cu") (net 2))
 (segment (start 92.043489 99.165489) (end 89.132489 99.165489) (width 0.25) (layer "B.Cu") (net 2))
 (segment (start 60.0225 100.457) (end 60.0225 98.2145) (width 0.25) (layer "F.Cu") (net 7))
 (segment (start 60.0225 98.2145) (end 61.331 96.906) (width 0.25) (layer "F.Cu") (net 7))
 (segment (start 59.657 96.906) (end 56.614 99.949) (width 0.25) (layer "F.Cu") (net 7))
 (segment (start 61.331 96.906) (end 59.657 96.906) (width 0.25) (layer "F.Cu") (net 7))
 (segment (start 79.723 96.906) (end 81.397 96.906) (width 0.25) (layer "F.Cu") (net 5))
 (segment (start 80.0885 98.2145) (end 81.397 96.906) (width 0.25) (layer "F.Cu") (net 5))
 (segment (start 80.0885 100.33) (end 80.0885 98.2145) (width 0.25) (layer "F.Cu") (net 5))
 (segment (start 76.68 99.949) (end 79.723 96.906) (width 0.25) (layer "F.Cu") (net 5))
 (segment (start 90.19 116.188) (end 90.19 115.717) (width 1) (layer "F.Cu") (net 4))
 (segment (start 90.19 115.717) (end 85.217 110.744) (width 1) (layer "F.Cu") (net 4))
 (segment (start 69.088 112.157) (end 69.088 116.952) (width 0.25) (layer "F.Cu") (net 11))
 (segment (start 69.088 116.952) (end 67.828 118.212) (width 0.25) (layer "F.Cu") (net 11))
 (segment (start 69.088 106.807) (end 69.088 112.157) (width 0.25) (layer "F.Cu") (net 11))
 (segment (start 86.832489 112.049511) (end 83.439 115.443) (width 1) (layer "B.Cu") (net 11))
 (segment (start 67.828 116.322) (end 67.828 118.212) (width 1) (layer "B.Cu") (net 11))
 (segment (start 68.707 115.443) (end 67.828 116.322) (width 1) (layer "B.Cu") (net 11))
 (segment (start 83.439 115.443) (end 68.707 115.443) (width 1) (layer "B.Cu") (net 11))
 (segment (start 93.218 110.5) (end 91.668489 112.049511) (width 1) (layer "B.Cu") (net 11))
 (segment (start 91.668489 112.049511) (end 86.832489 112.049511) (width 1) (layer "B.Cu") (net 11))
 (segment (start 94.842022 107.044022) (end 94.842022 113.341) (width 0.25) (layer "B.Cu") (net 12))
 (segment (start 81.654489 119.386511) (end 74.082511 119.386511) (width 0.25) (layer "B.Cu") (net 12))
 (segment (start 86.17752 114.86348) (end 81.654489 119.386511) (width 0.25) (layer "B.Cu") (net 12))
 (segment (start 74.082511 119.386511) (end 72.908 118.212) (width 0.25) (layer "B.Cu") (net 12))
 (segment (start 93.319542 114.86348) (end 86.17752 114.86348) (width 0.25) (layer "B.Cu") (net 12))
 (segment (start 94.842022 113.341) (end 93.319542 114.86348) (width 0.25) (layer "B.Cu") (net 12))
 (segment (start 93.218 105.42) (end 94.842022 107.044022) (width 0.25) (layer "B.Cu") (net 12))
 (segment (start 85.991326 114.41397) (end 82.193296 118.212) (width 0.25) (layer "B.Cu") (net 13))
 (segment (start 94.392511 112.236489) (end 92.21503 114.41397) (width 0.25) (layer "B.Cu") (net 13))
 (segment (start 92.21503 114.41397) (end 85.991326 114.41397) (width 0.25) (layer "B.Cu") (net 13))
 (segment (start 93.218 107.96) (end 93.609 107.96) (width 0.25) (layer "B.Cu") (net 13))
 (segment (start 93.609 107.96) (end 94.392511 108.743511) (width 0.25) (layer "B.Cu") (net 13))
 (segment (start 94.392511 108.743511) (end 94.392511 112.236489) (width 0.25) (layer "B.Cu") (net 13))
 (segment (start 82.193296 118.212) (end 75.448 118.212) (width 0.25) (layer "B.Cu") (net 13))
 (segment (start 75.204 73.008) (end 75.204 74.95) (width 1) (layer "F.Cu") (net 8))
 (segment (start 75.204 74.95) (end 79.38 79.126) (width 1) (layer "F.Cu") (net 8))
 (segment (start 79.38 79.126) (end 81.397 79.126) (width 1) (layer "F.Cu") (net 8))
 (segment (start 52.892 78.307) (end 52.892 73.135) (width 1) (layer "F.Cu") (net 3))
 (segment (start 81.397 86.746) (end 61.331 86.746) (width 1) (layer "F.Cu") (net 3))
 (segment (start 61.331 86.746) (end 52.892 78.307) (width 1) (layer "F.Cu") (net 3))
 (segment (start 76.708 109.408) (end 81.870511 104.245489) (width 0.25) (layer "F.Cu") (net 10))
 (segment (start 71.628 106.807) (end 74.229 109.408) (width 0.25) (layer "F.Cu") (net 10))
 (segment (start 71.628 106.807) (end 71.628 112.157) (width 0.25) (layer "F.Cu") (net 10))
 (segment (start 81.870511 104.245489) (end 91.852511 104.245489) (width 0.25) (layer "F.Cu") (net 10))
 (segment (start 76.962 110.681) (end 76.962 109.662) (width 0.25) (layer "F.Cu") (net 10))
 (segment (start 76.962 109.662) (end 76.708 109.408) (width 0.25) (layer "F.Cu") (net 10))
 (segment (start 74.229 109.408) (end 76.708 109.408) (width 0.25) (layer "F.Cu") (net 10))
 (segment (start 91.852511 104.245489) (end 93.218 102.88) (width 0.25) (layer "F.Cu") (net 10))
 (segment (start 90.001489 98.974511) (end 86.95748 102.01852) (width 0.25) (layer "F.Cu") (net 16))
 (segment (start 93.218 97.8) (end 92.043489 98.974511) (width 0.25) (layer "F.Cu") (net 16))
 (segment (start 66.14052 102.01852) (end 86.95748 102.01852) (width 0.25) (layer "F.Cu") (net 16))
 (segment (start 92.043489 98.974511) (end 90.001489 98.974511) (width 0.25) (layer "F.Cu") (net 16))
 (segment (start 65.468 101.346) (end 66.14052 102.01852) (width 0.25) (layer "F.Cu") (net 16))
 (segment (start 63.818 101.346) (end 61.9585 101.346) (width 0.25) (layer "F.Cu") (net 6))
 (segment (start 61.9585 101.346) (end 61.8975 101.407) (width 0.25) (layer "F.Cu") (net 6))
 (segment (start 84.077 101.28) (end 84.138 101.219) (width 0.25) (layer "F.Cu") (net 18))
 (segment (start 81.9635 101.28) (end 84.077 101.28) (width 0.25) (layer "F.Cu") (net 18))
 (segment (start 61.508 78.949) (end 61.331 79.126) (width 1) (layer "F.Cu") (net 9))
 (segment (start 61.508 73.152) (end 61.508 78.949) (width 1) (layer "F.Cu") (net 9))
 (segment (start 92.043489 96.434511) (end 90.382489 96.434511) (width 0.25) (layer "F.Cu") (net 17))
 (segment (start 90.382489 96.434511) (end 85.788 101.029) (width 0.25) (layer "F.Cu") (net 17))
 (segment (start 93.218 95.26) (end 92.043489 96.434511) (width 0.25) (layer "F.Cu") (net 17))
 (segment (start 85.788 101.029) (end 85.788 101.219) (width 0.25) (layer "F.Cu") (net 17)))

